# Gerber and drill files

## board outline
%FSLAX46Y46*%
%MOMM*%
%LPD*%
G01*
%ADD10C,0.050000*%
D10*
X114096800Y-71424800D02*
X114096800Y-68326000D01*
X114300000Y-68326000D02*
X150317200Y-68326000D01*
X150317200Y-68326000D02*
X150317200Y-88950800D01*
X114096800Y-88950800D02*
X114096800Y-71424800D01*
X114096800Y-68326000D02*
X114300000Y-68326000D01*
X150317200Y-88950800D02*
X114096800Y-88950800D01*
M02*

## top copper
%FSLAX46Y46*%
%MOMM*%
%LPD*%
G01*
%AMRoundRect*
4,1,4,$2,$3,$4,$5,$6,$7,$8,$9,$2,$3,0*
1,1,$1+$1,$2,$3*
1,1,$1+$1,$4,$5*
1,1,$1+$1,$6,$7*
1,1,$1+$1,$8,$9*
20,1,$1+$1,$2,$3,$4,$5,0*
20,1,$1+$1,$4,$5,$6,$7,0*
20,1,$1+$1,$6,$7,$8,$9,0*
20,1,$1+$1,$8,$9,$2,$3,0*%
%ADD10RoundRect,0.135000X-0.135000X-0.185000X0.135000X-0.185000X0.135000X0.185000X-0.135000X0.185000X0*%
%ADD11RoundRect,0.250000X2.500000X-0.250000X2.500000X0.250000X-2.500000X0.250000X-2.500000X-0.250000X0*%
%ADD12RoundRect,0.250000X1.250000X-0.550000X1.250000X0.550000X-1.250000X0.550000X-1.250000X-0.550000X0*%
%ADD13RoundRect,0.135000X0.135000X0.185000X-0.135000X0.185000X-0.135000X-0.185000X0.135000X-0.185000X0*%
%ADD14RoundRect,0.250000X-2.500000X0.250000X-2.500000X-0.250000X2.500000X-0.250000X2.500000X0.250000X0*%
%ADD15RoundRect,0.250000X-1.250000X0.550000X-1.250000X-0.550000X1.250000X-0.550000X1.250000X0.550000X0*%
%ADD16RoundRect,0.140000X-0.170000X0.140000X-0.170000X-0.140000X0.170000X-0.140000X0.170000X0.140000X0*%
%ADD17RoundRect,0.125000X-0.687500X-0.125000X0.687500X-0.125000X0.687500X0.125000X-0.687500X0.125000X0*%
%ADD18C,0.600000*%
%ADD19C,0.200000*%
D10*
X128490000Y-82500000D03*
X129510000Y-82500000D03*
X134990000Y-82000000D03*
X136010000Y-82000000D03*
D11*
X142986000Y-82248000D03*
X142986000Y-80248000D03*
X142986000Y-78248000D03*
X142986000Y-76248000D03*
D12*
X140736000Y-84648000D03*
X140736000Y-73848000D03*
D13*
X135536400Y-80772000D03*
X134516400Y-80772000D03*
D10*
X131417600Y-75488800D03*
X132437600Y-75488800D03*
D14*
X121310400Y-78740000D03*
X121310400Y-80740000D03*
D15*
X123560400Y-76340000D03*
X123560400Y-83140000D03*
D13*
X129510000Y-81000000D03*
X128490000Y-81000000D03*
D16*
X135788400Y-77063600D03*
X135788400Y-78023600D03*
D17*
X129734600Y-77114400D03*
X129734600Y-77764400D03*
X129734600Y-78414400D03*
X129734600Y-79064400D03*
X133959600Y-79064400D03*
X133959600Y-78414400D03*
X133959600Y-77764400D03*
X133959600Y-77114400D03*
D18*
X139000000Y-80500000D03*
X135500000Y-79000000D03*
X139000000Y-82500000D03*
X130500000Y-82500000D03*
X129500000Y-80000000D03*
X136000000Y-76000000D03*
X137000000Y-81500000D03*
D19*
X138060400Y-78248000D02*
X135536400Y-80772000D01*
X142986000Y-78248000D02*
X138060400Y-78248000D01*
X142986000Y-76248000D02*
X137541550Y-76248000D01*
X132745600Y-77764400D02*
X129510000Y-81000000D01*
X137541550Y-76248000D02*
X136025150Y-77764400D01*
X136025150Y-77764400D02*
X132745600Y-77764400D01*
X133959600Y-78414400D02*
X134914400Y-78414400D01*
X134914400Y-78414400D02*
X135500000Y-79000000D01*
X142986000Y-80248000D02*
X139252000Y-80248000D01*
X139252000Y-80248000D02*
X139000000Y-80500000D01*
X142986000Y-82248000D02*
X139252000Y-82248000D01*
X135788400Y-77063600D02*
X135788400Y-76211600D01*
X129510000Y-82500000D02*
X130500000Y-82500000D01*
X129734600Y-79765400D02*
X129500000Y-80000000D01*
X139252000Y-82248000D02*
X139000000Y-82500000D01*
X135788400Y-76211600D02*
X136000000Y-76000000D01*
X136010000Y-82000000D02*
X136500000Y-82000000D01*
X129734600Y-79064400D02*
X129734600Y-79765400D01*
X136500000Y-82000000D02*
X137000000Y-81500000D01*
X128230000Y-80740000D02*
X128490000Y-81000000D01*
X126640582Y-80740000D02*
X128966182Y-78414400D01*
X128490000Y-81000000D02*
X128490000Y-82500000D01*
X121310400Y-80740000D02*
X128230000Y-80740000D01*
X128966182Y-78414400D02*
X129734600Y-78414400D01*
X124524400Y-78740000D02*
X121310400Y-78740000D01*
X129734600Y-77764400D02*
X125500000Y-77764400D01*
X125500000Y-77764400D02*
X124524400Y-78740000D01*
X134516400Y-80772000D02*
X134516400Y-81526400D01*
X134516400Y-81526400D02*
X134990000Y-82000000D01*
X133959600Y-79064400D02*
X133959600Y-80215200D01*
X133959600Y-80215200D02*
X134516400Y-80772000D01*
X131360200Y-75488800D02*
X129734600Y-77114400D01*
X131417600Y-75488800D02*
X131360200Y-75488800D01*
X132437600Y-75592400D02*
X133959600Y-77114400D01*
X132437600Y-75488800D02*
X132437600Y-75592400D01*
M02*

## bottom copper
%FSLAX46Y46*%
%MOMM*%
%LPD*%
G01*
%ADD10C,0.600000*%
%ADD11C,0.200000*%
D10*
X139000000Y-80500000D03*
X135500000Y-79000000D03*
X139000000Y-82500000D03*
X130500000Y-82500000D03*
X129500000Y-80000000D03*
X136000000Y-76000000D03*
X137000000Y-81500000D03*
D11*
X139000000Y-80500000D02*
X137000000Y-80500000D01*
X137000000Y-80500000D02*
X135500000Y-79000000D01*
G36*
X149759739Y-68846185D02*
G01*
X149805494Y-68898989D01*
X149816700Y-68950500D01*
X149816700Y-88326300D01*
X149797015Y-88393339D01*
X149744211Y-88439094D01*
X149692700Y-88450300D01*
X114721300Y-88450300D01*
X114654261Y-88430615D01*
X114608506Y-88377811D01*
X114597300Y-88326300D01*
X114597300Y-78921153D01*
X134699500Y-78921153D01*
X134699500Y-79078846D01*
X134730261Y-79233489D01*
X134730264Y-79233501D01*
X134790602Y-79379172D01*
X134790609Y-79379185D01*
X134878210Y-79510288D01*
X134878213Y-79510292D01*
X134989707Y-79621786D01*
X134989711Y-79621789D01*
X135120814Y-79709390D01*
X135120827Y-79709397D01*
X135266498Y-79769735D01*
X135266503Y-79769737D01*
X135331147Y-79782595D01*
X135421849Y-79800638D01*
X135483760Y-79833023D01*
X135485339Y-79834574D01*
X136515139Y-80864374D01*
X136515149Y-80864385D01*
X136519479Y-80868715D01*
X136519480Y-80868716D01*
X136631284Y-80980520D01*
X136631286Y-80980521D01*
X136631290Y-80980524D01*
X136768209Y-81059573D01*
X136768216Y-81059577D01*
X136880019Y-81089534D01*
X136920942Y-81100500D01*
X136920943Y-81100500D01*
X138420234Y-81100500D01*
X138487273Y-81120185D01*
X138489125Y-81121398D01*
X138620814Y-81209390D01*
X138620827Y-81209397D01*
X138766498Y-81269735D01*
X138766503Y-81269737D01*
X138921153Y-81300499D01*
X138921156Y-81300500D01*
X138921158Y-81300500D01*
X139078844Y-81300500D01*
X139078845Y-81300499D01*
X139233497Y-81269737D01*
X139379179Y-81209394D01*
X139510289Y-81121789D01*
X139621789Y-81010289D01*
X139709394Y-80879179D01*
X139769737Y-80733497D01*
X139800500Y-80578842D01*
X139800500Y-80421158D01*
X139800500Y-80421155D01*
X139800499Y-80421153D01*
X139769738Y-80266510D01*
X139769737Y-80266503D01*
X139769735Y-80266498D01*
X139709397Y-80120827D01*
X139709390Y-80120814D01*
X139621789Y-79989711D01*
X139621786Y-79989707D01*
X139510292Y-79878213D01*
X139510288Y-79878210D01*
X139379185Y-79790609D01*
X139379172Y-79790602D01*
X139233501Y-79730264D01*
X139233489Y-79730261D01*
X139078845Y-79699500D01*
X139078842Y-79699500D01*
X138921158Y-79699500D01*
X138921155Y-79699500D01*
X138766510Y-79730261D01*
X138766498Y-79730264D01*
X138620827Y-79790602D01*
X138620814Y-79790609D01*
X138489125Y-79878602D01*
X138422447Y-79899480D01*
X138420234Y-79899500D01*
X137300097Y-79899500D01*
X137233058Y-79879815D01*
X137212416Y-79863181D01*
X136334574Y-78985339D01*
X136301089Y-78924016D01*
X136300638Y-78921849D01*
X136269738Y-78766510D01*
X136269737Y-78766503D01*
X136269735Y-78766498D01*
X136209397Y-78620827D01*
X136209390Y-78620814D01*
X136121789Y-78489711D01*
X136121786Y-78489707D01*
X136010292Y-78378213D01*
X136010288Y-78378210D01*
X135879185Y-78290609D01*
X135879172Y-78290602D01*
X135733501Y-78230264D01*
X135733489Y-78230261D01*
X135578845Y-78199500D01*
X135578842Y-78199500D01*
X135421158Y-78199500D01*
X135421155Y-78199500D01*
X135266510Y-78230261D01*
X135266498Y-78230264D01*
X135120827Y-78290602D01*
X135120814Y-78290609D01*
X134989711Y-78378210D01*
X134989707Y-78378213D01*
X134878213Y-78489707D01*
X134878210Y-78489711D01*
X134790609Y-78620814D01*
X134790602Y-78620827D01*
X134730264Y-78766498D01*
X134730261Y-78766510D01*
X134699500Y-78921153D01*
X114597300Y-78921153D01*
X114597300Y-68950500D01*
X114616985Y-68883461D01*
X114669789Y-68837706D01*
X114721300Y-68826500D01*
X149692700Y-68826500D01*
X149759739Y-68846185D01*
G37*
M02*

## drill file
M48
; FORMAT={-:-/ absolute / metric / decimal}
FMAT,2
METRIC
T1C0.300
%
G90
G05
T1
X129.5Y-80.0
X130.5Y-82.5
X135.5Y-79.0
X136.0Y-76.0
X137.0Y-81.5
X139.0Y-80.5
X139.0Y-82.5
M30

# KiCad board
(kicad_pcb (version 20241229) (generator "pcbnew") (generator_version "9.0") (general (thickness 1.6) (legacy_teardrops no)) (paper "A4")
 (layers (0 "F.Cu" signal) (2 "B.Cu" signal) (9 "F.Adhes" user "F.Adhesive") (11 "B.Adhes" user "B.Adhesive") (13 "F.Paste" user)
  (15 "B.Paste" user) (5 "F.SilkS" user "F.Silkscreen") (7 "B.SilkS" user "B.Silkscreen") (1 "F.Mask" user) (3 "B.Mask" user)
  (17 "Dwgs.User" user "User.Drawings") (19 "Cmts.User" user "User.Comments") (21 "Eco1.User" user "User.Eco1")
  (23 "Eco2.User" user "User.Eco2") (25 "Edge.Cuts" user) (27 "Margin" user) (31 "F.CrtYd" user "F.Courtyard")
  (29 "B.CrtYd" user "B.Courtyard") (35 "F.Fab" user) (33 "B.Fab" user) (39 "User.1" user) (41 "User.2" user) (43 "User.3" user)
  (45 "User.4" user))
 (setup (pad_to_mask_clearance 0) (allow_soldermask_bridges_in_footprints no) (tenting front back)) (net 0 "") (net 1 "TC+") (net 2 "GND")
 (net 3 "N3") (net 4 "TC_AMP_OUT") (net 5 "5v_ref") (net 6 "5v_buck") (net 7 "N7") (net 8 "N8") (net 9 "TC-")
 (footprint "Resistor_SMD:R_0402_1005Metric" (layer "F.Cu") (at 129 82.5)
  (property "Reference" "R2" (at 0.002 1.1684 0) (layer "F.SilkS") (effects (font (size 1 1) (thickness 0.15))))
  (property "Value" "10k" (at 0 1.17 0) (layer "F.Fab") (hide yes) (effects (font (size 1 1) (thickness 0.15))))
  (pad "1" smd roundrect (at -0.51 0) (size 0.54 0.64) (layers "F.Cu" "F.Mask" "F.Paste") (roundrect_rratio 0.25) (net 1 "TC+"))
  (pad "2" smd roundrect (at 0.51 0) (size 0.54 0.64) (layers "F.Cu" "F.Mask" "F.Paste") (roundrect_rratio 0.25) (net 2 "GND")))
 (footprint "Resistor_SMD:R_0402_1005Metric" (layer "F.Cu") (at 135.5 82)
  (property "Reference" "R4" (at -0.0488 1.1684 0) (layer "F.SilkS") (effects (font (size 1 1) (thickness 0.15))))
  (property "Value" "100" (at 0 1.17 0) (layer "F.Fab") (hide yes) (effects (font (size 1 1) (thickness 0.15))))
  (pad "1" smd roundrect (at -0.51 0) (size 0.54 0.64) (layers "F.Cu" "F.Mask" "F.Paste") (roundrect_rratio 0.25) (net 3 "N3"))
  (pad "2" smd roundrect (at 0.51 0) (size 0.54 0.64) (layers "F.Cu" "F.Mask" "F.Paste") (roundrect_rratio 0.25) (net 2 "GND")))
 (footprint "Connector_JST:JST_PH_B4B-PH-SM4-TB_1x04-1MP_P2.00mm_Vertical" (layer "F.Cu") (at 142.486 79.248 90)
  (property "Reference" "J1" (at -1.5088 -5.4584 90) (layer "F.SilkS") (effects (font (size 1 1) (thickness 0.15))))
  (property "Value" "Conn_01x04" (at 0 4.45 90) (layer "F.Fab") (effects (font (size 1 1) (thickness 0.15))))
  (pad "1" smd roundrect (at -3 0.5 90) (size 1 5.5) (layers "F.Cu" "F.Mask" "F.Paste") (roundrect_rratio 0.25) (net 2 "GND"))
  (pad "2" smd roundrect (at -1 0.5 90) (size 1 5.5) (layers "F.Cu" "F.Mask" "F.Paste") (roundrect_rratio 0.25) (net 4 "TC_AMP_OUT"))
  (pad "3" smd roundrect (at 1 0.5 90) (size 1 5.5) (layers "F.Cu" "F.Mask" "F.Paste") (roundrect_rratio 0.25) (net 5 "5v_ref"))
  (pad "4" smd roundrect (at 3 0.5 90) (size 1 5.5) (layers "F.Cu" "F.Mask" "F.Paste") (roundrect_rratio 0.25) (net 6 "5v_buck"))
  (pad "MP" smd roundrect (at -5.4 -1.75 90) (size 1.6 3) (layers "F.Cu" "F.Mask" "F.Paste") (roundrect_rratio 0.15625))
  (pad "MP" smd roundrect (at 5.4 -1.75 90) (size 1.6 3) (layers "F.Cu" "F.Mask" "F.Paste") (roundrect_rratio 0.15625)))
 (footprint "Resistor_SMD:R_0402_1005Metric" (layer "F.Cu") (at 135.0264 80.772 180)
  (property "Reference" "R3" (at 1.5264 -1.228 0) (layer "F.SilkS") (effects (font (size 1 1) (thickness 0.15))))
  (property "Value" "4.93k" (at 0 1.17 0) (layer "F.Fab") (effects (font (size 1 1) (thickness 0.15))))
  (pad "1" smd roundrect (at -0.51 0 180) (size 0.54 0.64) (layers "F.Cu" "F.Mask" "F.Paste") (roundrect_rratio 0.25) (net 5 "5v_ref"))
  (pad "2" smd roundrect (at 0.51 0 180) (size 0.54 0.64) (layers "F.Cu" "F.Mask" "F.Paste") (roundrect_rratio 0.25) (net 3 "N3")))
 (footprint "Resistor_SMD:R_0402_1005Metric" (layer "F.Cu") (at 131.9276 75.4888)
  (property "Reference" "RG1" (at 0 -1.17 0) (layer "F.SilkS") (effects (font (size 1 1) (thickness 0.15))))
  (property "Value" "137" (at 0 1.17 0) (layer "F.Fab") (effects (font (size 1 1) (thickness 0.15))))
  (pad "1" smd roundrect (at -0.51 0) (size 0.54 0.64) (layers "F.Cu" "F.Mask" "F.Paste") (roundrect_rratio 0.25) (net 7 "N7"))
  (pad "2" smd roundrect (at 0.51 0) (size 0.54 0.64) (layers "F.Cu" "F.Mask" "F.Paste") (roundrect_rratio 0.25) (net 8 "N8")))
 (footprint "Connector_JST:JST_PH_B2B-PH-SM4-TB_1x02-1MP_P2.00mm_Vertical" (layer "F.Cu") (at 121.8104 79.74 -90)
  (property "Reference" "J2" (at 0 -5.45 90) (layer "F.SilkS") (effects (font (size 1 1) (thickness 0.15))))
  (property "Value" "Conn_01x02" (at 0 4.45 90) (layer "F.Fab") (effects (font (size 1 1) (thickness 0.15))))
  (pad "1" smd roundrect (at -1 0.5 270) (size 1 5.5) (layers "F.Cu" "F.Mask" "F.Paste") (roundrect_rratio 0.25) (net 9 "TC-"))
  (pad "2" smd roundrect (at 1 0.5 270) (size 1 5.5) (layers "F.Cu" "F.Mask" "F.Paste") (roundrect_rratio 0.25) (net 1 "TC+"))
  (pad "MP" smd roundrect (at -3.4 -1.75 270) (size 1.6 3) (layers "F.Cu" "F.Mask" "F.Paste") (roundrect_rratio 0.15625))
  (pad "MP" smd roundrect (at 3.4 -1.75 270) (size 1.6 3) (layers "F.Cu" "F.Mask" "F.Paste") (roundrect_rratio 0.15625)))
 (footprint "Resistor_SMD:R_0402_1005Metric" (layer "F.Cu") (at 129 81 180)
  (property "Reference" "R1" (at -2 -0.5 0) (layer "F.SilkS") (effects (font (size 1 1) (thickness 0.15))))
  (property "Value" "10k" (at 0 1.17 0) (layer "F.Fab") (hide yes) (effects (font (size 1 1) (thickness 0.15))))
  (pad "1" smd roundrect (at -0.51 0 180) (size 0.54 0.64) (layers "F.Cu" "F.Mask" "F.Paste") (roundrect_rratio 0.25) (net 6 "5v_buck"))
  (pad "2" smd roundrect (at 0.51 0 180) (size 0.54 0.64) (layers "F.Cu" "F.Mask" "F.Paste") (roundrect_rratio 0.25) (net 1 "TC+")))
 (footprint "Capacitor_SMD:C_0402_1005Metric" (layer "F.Cu") (at 135.7884 77.5436 -90)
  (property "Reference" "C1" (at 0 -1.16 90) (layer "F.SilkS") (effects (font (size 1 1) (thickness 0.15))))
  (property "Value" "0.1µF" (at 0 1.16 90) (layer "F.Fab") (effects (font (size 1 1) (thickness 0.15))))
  (pad "1" smd roundrect (at -0.48 0 270) (size 0.56 0.62) (layers "F.Cu" "F.Mask" "F.Paste") (roundrect_rratio 0.25) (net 2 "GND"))
  (pad "2" smd roundrect (at 0.48 0 270) (size 0.56 0.62) (layers "F.Cu" "F.Mask" "F.Paste") (roundrect_rratio 0.25) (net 6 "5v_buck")))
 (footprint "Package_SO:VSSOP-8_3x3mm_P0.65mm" (layer "F.Cu") (at 131.8471 78.0894)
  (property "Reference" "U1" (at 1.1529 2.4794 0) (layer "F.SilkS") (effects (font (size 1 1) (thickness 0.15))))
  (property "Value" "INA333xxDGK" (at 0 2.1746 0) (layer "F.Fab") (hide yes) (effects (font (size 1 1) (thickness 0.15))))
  (pad "1" smd roundrect (at -2.1125 -0.975) (size 1.625 0.5) (layers "F.Cu" "F.Mask" "F.Paste") (roundrect_rratio 0.25) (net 7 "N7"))
  (pad "2" smd roundrect (at -2.1125 -0.325) (size 1.625 0.5) (layers "F.Cu" "F.Mask" "F.Paste") (roundrect_rratio 0.25) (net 9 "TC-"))
  (pad "3" smd roundrect (at -2.1125 0.325) (size 1.625 0.5) (layers "F.Cu" "F.Mask" "F.Paste") (roundrect_rratio 0.25) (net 1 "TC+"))
  (pad "4" smd roundrect (at -2.1125 0.975) (size 1.625 0.5) (layers "F.Cu" "F.Mask" "F.Paste") (roundrect_rratio 0.25) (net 2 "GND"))
  (pad "5" smd roundrect (at 2.1125 0.975) (size 1.625 0.5) (layers "F.Cu" "F.Mask" "F.Paste") (roundrect_rratio 0.25) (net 3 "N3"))
  (pad "6" smd roundrect (at 2.1125 0.325) (size 1.625 0.5) (layers "F.Cu" "F.Mask" "F.Paste") (roundrect_rratio 0.25) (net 4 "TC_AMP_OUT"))
  (pad "7" smd roundrect (at 2.1125 -0.325) (size 1.625 0.5) (layers "F.Cu" "F.Mask" "F.Paste") (roundrect_rratio 0.25) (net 6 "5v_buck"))
  (pad "8" smd roundrect (at 2.1125 -0.975) (size 1.625 0.5) (layers "F.Cu" "F.Mask" "F.Paste") (roundrect_rratio 0.25) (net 8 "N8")))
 (gr_line (start 114.0968 71.4248) (end 114.0968 68.326) (stroke (width 0.05) (type default)) (layer "Edge.Cuts"))
 (gr_line (start 114.3 68.326) (end 150.3172 68.326) (stroke (width 0.05) (type default)) (layer "Edge.Cuts"))
 (gr_line (start 150.3172 68.326) (end 150.3172 88.9508) (stroke (width 0.05) (type default)) (layer "Edge.Cuts"))
 (gr_line (start 114.0968 88.9508) (end 114.0968 71.4248) (stroke (width 0.05) (type default)) (layer "Edge.Cuts"))
 (gr_line (start 114.0968 68.326) (end 114.3 68.326) (stroke (width 0.05) (type default)) (layer "Edge.Cuts"))
 (gr_line (start 150.3172 88.9508) (end 114.0968 88.9508) (stroke (width 0.05) (type default)) (layer "Edge.Cuts"))
 (segment (start 138.0604 78.248) (end 135.5364 80.772) (width 0.2) (layer "F.Cu") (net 5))
 (segment (start 142.986 78.248) (end 138.0604 78.248) (width 0.2) (layer "F.Cu") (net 5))
 (segment (start 142.986 76.248) (end 137.54155 76.248) (width 0.2) (layer "F.Cu") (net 6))
 (segment (start 132.7456 77.7644) (end 129.51 81) (width 0.2) (layer "F.Cu") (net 6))
 (segment (start 137.54155 76.248) (end 136.02515 77.7644) (width 0.2) (layer "F.Cu") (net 6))
 (segment (start 136.02515 77.7644) (end 132.7456 77.7644) (width 0.2) (layer "F.Cu") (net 6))
 (segment (start 133.9596 78.4144) (end 134.9144 78.4144) (width 0.2) (layer "F.Cu") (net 4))
 (segment (start 134.9144 78.4144) (end 135.5 79) (width 0.2) (layer "F.Cu") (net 4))
 (segment (start 142.986 80.248) (end 139.252 80.248) (width 0.2) (layer "F.Cu") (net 4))
 (segment (start 139.252 80.248) (end 139 80.5) (width 0.2) (layer "F.Cu") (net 4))
 (via (at 139 80.5) (size 0.6) (drill 0.3) (layers "F.Cu" "B.Cu") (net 4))
 (via (at 135.5 79) (size 0.6) (drill 0.3) (layers "F.Cu" "B.Cu") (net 4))
 (segment (start 139 80.5) (end 137 80.5) (width 0.2) (layer "B.Cu") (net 4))
 (segment (start 137 80.5) (end 135.5 79) (width 0.2) (layer "B.Cu") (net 4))
 (segment (start 142.986 82.248) (end 139.252 82.248) (width 0.2) (layer "F.Cu") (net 2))
 (segment (start 135.7884 77.0636) (end 135.7884 76.2116) (width 0.2) (layer "F.Cu") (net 2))
 (segment (start 129.51 82.5) (end 130.5 82.5) (width 0.2) (layer "F.Cu") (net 2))
 (segment (start 129.7346 79.7654) (end 129.5 80) (width 0.2) (layer "F.Cu") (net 2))
 (segment (start 139.252 82.248) (end 139 82.5) (width 0.2) (layer "F.Cu") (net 2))
 (segment (start 135.7884 76.2116) (end 136 76) (width 0.2) (layer "F.Cu") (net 2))
 (segment (start 136.01 82) (end 136.5 82) (width 0.2) (layer "F.Cu") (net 2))
 (segment (start 129.7346 79.0644) (end 129.7346 79.7654) (width 0.2) (layer "F.Cu") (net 2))
 (segment (start 136.5 82) (end 137 81.5) (width 0.2) (layer "F.Cu") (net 2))
 (via (at 139 82.5) (size 0.6) (drill 0.3) (layers "F.Cu" "B.Cu") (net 2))
 (via (at 130.5 82.5) (size 0.6) (drill 0.3) (layers "F.Cu" "B.Cu") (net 2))
 (via (at 129.5 80) (size 0.6) (drill 0.3) (layers "F.Cu" "B.Cu") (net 2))
 (via (at 136 76) (size 0.6) (drill 0.3) (layers "F.Cu" "B.Cu") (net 2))
 (via (at 137 81.5) (size 0.6) (drill 0.3) (layers "F.Cu" "B.Cu") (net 2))
 (segment (start 128.23 80.74) (end 128.49 81) (width 0.2) (layer "F.Cu") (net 1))
 (segment (start 126.640582 80.74) (end 128.966182 78.4144) (width 0.2) (layer "F.Cu") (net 1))
 (segment (start 128.49 81) (end 128.49 82.5) (width 0.2) (layer "F.Cu") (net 1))
 (segment (start 121.3104 80.74) (end 128.23 80.74) (width 0.2) (layer "F.Cu") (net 1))
 (segment (start 128.966182 78.4144) (end 129.7346 78.4144) (width 0.2) (layer "F.Cu") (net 1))
 (segment (start 124.5244 78.74) (end 121.3104 78.74) (width 0.2) (layer "F.Cu") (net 9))
 (segment (start 129.7346 77.7644) (end 125.5 77.7644) (width 0.2) (layer "F.Cu") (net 9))
 (segment (start 125.5 77.7644) (end 124.5244 78.74) (width 0.2) (layer "F.Cu") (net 9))
 (segment (start 134.5164 80.772) (end 134.5164 81.5264) (width 0.2) (layer "F.Cu") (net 3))
 (segment (start 134.5164 81.5264) (end 134.99 82) (width 0.2) (layer "F.Cu") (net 3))
 (segment (start 133.9596 79.0644) (end 133.9596 80.2152) (width 0.2) (layer "F.Cu") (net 3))
 (segment (start 133.9596 80.2152) (end 134.5164 80.772) (width 0.2) (layer "F.Cu") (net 3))
 (segment (start 131.3602 75.4888) (end 129.7346 77.1144) (width 0.2) (layer "F.Cu") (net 7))
 (segment (start 131.4176 75.4888) (end 131.3602 75.4888) (width 0.2) (layer "F.Cu") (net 7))
 (segment (start 132.4376 75.5924) (end 133.9596 77.1144) (width 0.2) (layer "F.Cu") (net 8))
 (segment (start 132.4376 75.4888) (end 132.4376 75.5924) (width 0.2) (layer "F.Cu") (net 8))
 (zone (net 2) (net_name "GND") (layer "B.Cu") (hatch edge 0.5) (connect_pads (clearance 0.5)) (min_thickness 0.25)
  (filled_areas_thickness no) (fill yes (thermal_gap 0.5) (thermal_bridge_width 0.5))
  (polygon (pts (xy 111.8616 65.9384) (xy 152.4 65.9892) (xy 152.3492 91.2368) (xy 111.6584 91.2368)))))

